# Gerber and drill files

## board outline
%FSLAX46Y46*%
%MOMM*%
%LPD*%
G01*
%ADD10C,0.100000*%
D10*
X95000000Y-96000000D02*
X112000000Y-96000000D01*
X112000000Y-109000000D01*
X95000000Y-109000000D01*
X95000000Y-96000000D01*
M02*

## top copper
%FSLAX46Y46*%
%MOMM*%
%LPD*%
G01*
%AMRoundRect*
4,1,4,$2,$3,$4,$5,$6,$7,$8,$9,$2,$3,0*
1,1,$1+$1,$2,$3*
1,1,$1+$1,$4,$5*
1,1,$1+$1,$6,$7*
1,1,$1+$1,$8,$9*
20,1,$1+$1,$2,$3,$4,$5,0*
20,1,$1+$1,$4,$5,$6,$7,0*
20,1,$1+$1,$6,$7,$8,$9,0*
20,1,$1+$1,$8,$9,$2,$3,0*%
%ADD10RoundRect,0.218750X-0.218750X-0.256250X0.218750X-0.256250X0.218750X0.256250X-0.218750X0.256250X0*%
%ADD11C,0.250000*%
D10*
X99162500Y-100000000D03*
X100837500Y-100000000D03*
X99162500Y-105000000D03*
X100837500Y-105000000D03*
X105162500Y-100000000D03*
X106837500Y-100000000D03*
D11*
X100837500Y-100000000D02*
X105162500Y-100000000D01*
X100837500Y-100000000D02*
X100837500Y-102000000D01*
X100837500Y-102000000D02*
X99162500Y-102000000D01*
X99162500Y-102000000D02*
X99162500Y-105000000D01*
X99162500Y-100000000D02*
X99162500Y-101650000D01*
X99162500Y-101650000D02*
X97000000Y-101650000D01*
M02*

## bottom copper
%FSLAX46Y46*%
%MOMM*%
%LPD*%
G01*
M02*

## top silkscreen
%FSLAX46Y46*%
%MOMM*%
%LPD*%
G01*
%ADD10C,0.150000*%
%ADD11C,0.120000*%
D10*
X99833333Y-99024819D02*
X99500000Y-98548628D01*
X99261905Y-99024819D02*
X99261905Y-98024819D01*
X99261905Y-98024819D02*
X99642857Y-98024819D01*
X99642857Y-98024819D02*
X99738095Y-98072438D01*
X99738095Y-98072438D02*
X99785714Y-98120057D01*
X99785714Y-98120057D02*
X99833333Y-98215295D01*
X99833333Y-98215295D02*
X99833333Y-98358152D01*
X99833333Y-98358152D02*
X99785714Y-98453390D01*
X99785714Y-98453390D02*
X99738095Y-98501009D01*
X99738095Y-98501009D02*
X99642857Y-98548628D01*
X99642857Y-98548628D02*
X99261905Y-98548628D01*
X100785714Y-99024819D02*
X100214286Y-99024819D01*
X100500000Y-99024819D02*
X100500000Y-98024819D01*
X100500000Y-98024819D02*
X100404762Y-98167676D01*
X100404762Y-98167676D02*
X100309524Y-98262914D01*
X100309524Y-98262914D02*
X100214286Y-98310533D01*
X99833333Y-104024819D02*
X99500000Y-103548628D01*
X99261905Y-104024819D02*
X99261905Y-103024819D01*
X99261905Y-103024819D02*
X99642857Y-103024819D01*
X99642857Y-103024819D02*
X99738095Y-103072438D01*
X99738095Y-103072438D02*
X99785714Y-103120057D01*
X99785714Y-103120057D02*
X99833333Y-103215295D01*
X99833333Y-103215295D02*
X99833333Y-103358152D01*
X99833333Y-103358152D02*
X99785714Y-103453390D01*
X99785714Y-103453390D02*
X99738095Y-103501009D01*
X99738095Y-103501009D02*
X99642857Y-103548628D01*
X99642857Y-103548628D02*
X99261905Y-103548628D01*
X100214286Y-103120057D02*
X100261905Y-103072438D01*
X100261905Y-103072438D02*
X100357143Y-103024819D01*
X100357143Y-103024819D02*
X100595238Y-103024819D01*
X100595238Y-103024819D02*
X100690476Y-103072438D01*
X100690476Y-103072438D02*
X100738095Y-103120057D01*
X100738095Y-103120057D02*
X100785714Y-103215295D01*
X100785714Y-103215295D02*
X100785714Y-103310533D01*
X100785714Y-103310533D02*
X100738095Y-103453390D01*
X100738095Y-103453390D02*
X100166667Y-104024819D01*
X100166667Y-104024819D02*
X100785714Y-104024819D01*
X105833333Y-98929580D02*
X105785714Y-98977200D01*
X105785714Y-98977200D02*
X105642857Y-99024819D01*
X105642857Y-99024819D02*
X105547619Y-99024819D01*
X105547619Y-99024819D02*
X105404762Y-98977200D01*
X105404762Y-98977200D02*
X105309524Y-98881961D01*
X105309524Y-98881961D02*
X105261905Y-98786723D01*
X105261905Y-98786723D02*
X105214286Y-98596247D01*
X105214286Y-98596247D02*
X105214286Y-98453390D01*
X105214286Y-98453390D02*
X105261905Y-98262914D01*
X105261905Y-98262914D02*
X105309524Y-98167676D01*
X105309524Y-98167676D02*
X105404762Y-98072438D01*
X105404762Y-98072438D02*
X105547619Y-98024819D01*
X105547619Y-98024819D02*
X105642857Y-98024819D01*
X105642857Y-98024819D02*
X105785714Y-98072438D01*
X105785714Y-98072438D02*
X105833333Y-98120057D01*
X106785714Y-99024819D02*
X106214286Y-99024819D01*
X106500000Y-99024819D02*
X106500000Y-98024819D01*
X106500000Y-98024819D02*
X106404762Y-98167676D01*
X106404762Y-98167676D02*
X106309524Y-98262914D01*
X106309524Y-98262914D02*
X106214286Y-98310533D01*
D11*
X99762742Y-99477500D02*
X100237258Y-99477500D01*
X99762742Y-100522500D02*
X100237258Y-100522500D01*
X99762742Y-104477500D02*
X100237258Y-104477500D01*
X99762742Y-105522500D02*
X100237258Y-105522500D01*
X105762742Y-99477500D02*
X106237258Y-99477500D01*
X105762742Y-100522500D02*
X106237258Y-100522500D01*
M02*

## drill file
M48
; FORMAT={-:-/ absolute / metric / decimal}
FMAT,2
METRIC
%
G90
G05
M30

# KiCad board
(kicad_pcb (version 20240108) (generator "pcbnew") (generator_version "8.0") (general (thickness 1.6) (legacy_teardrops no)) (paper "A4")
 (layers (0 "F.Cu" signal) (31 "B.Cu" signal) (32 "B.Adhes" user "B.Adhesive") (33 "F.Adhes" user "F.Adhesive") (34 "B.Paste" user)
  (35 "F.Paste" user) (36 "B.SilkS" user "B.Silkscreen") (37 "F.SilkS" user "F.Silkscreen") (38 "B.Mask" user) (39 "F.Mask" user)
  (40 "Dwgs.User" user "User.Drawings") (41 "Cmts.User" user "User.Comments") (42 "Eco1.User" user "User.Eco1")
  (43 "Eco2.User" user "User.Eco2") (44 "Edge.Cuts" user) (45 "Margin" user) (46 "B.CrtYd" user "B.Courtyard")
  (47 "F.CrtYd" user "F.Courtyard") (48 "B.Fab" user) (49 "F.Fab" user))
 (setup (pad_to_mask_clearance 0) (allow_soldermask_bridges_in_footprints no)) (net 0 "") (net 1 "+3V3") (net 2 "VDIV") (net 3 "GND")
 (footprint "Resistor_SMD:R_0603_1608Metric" (layer "F.Cu") (at 100 100)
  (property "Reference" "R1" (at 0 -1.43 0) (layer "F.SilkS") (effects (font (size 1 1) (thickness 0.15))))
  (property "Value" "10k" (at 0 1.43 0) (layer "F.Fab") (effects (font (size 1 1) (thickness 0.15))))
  (fp_line (start -0.237258 -0.5225) (end 0.237258 -0.5225) (stroke (width 0.12) (type solid)) (layer "F.SilkS"))
  (fp_line (start -0.237258 0.5225) (end 0.237258 0.5225) (stroke (width 0.12) (type solid)) (layer "F.SilkS"))
  (pad "1" smd roundrect (at -0.8375 0) (size 0.875 0.95) (layers "F.Cu" "F.Paste" "F.Mask") (roundrect_rratio 0.25) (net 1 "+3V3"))
  (pad "2" smd roundrect (at 0.8375 0) (size 0.875 0.95) (layers "F.Cu" "F.Paste" "F.Mask") (roundrect_rratio 0.25) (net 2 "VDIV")))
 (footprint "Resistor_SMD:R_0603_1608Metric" (layer "F.Cu") (at 100 105)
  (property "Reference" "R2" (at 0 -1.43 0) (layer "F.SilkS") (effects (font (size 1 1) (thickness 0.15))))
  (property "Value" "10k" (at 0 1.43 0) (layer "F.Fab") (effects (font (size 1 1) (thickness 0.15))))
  (fp_line (start -0.237258 -0.5225) (end 0.237258 -0.5225) (stroke (width 0.12) (type solid)) (layer "F.SilkS"))
  (fp_line (start -0.237258 0.5225) (end 0.237258 0.5225) (stroke (width 0.12) (type solid)) (layer "F.SilkS"))
  (pad "1" smd roundrect (at -0.8375 0) (size 0.875 0.95) (layers "F.Cu" "F.Paste" "F.Mask") (roundrect_rratio 0.25) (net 2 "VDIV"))
  (pad "2" smd roundrect (at 0.8375 0) (size 0.875 0.95) (layers "F.Cu" "F.Paste" "F.Mask") (roundrect_rratio 0.25) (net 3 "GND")))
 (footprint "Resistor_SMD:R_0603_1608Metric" (layer "F.Cu") (at 106 100)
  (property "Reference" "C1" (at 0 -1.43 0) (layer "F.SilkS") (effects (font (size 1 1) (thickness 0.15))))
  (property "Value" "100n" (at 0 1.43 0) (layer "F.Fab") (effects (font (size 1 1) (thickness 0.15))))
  (fp_line (start -0.237258 -0.5225) (end 0.237258 -0.5225) (stroke (width 0.12) (type solid)) (layer "F.SilkS"))
  (fp_line (start -0.237258 0.5225) (end 0.237258 0.5225) (stroke (width 0.12) (type solid)) (layer "F.SilkS"))
  (pad "1" smd roundrect (at -0.8375 0) (size 0.875 0.95) (layers "F.Cu" "F.Paste" "F.Mask") (roundrect_rratio 0.25) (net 2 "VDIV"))
  (pad "2" smd roundrect (at 0.8375 0) (size 0.875 0.95) (layers "F.Cu" "F.Paste" "F.Mask") (roundrect_rratio 0.25) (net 3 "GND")))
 (segment (start 100.8375 100) (end 105.1625 100) (width 0.25) (layer "F.Cu") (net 2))
 (segment (start 100.8375 100) (end 100.8375 102.0) (width 0.25) (layer "F.Cu") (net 2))
 (segment (start 100.8375 102.0) (end 99.1625 102.0) (width 0.25) (layer "F.Cu") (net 2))
 (segment (start 99.1625 102.0) (end 99.1625 105) (width 0.25) (layer "F.Cu") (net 2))
 (segment (start 99.1625 100) (end 99.1625 101.65) (width 0.25) (layer "F.Cu") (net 1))
 (segment (start 99.1625 101.65) (end 97.0 101.65) (width 0.25) (layer "F.Cu") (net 1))
 (gr_rect (start 95 96) (end 112 109) (stroke (width 0.1) (type default)) (fill none) (layer "Edge.Cuts")))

